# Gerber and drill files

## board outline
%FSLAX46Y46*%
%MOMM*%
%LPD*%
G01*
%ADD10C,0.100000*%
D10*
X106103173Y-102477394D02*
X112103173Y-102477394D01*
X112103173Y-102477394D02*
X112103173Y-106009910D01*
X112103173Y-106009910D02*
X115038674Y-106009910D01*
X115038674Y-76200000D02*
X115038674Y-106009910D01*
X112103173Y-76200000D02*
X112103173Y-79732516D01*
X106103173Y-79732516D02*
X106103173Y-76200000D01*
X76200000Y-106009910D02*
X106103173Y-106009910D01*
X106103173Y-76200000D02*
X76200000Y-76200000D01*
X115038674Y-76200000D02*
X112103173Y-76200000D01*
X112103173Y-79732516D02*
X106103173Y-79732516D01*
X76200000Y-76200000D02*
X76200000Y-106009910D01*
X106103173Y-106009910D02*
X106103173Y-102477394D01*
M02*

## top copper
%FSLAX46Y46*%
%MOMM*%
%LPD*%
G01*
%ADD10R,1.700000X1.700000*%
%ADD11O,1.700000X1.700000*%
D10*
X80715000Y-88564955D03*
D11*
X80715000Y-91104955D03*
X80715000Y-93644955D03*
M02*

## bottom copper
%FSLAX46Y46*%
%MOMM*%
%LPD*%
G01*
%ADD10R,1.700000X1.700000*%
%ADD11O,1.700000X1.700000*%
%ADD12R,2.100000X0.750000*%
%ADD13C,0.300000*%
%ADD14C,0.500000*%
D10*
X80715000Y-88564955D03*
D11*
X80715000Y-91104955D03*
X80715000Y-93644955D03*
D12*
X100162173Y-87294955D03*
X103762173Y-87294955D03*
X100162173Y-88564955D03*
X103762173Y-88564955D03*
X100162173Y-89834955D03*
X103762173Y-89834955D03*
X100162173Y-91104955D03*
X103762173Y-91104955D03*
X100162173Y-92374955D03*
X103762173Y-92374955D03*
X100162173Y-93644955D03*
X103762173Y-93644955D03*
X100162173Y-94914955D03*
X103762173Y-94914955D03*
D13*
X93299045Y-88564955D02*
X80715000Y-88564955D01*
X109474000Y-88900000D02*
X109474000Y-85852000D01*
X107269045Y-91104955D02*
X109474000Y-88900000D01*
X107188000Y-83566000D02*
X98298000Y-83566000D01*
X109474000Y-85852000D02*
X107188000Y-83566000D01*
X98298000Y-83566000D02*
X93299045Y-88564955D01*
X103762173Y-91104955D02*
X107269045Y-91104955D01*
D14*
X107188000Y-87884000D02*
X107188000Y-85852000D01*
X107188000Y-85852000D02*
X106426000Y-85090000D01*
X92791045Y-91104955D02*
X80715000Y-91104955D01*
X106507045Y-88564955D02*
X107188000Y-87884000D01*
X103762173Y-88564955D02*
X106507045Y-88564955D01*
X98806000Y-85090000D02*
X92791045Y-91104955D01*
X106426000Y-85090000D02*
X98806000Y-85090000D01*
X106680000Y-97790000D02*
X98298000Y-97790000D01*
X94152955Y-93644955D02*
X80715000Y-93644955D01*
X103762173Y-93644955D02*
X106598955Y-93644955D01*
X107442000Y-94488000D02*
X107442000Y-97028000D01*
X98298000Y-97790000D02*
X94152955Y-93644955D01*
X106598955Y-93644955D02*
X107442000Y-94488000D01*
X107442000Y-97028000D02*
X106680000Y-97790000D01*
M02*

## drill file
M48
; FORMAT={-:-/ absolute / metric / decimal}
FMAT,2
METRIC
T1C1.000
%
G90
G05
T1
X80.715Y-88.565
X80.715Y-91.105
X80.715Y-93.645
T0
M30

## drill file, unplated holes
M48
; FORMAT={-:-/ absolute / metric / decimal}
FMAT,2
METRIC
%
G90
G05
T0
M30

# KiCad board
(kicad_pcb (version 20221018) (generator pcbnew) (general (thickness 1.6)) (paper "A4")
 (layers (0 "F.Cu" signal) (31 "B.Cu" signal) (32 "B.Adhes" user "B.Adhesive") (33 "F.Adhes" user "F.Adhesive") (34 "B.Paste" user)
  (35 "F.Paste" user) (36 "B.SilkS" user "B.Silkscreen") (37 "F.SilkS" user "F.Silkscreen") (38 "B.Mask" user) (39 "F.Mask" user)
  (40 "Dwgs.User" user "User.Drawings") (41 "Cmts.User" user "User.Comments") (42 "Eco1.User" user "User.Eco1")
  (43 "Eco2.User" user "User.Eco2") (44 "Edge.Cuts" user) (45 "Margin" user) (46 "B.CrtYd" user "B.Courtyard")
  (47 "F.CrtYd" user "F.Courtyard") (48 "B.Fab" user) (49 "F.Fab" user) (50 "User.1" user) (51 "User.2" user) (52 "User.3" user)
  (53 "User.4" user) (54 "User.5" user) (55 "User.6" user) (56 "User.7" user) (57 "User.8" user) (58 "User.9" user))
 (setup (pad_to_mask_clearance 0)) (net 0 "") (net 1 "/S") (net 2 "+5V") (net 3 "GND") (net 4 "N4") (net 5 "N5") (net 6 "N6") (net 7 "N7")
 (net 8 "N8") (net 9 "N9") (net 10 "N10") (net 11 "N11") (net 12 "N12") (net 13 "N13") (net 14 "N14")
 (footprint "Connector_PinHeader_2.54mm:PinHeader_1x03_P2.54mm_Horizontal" (layer "F.Cu") (at 80.715 88.564955)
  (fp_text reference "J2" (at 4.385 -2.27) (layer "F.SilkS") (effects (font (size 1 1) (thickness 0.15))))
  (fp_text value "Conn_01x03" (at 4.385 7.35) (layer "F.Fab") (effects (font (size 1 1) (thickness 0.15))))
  (pad "1" thru_hole rect (at 0 0) (size 1.7 1.7) (drill 1) (layers "*.Cu" "*.Mask") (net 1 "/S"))
  (pad "2" thru_hole oval (at 0 2.54) (size 1.7 1.7) (drill 1) (layers "*.Cu" "*.Mask") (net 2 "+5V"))
  (pad "3" thru_hole oval (at 0 5.08) (size 1.7 1.7) (drill 1) (layers "*.Cu" "*.Mask") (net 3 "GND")))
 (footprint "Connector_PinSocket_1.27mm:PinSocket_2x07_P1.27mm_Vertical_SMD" (layer "B.Cu") (at 101.962173 91.104955 180)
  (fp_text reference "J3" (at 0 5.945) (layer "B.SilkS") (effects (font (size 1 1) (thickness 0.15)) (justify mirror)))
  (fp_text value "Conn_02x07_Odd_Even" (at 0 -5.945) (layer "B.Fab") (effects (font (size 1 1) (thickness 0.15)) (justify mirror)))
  (pad "1" smd rect (at 1.8 3.81 180) (size 2.1 0.75) (layers "B.Cu" "B.Paste" "B.Mask") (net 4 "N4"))
  (pad "2" smd rect (at -1.8 3.81 180) (size 2.1 0.75) (layers "B.Cu" "B.Paste" "B.Mask") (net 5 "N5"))
  (pad "3" smd rect (at 1.8 2.54 180) (size 2.1 0.75) (layers "B.Cu" "B.Paste" "B.Mask") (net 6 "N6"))
  (pad "4" smd rect (at -1.8 2.54 180) (size 2.1 0.75) (layers "B.Cu" "B.Paste" "B.Mask") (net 2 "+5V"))
  (pad "5" smd rect (at 1.8 1.27 180) (size 2.1 0.75) (layers "B.Cu" "B.Paste" "B.Mask") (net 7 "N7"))
  (pad "6" smd rect (at -1.8 1.27 180) (size 2.1 0.75) (layers "B.Cu" "B.Paste" "B.Mask") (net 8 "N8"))
  (pad "7" smd rect (at 1.8 0 180) (size 2.1 0.75) (layers "B.Cu" "B.Paste" "B.Mask") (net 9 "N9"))
  (pad "8" smd rect (at -1.8 0 180) (size 2.1 0.75) (layers "B.Cu" "B.Paste" "B.Mask") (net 1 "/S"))
  (pad "9" smd rect (at 1.8 -1.27 180) (size 2.1 0.75) (layers "B.Cu" "B.Paste" "B.Mask") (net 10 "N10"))
  (pad "10" smd rect (at -1.8 -1.27 180) (size 2.1 0.75) (layers "B.Cu" "B.Paste" "B.Mask") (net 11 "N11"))
  (pad "11" smd rect (at 1.8 -2.54 180) (size 2.1 0.75) (layers "B.Cu" "B.Paste" "B.Mask") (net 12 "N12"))
  (pad "12" smd rect (at -1.8 -2.54 180) (size 2.1 0.75) (layers "B.Cu" "B.Paste" "B.Mask") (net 3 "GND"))
  (pad "13" smd rect (at 1.8 -3.81 180) (size 2.1 0.75) (layers "B.Cu" "B.Paste" "B.Mask") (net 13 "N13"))
  (pad "14" smd rect (at -1.8 -3.81 180) (size 2.1 0.75) (layers "B.Cu" "B.Paste" "B.Mask") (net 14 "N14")))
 (gr_line (start 106.103173 102.477394) (end 112.103173 102.477394) (stroke (width 0.1) (type solid)) (layer "Edge.Cuts"))
 (gr_line (start 112.103173 102.477394) (end 112.103173 106.00991) (stroke (width 0.1) (type solid)) (layer "Edge.Cuts"))
 (gr_line (start 112.103173 106.00991) (end 115.038674 106.00991) (stroke (width 0.1) (type solid)) (layer "Edge.Cuts"))
 (gr_line (start 115.038674 76.2) (end 115.038674 106.00991) (stroke (width 0.1) (type solid)) (layer "Edge.Cuts"))
 (gr_line (start 112.103173 76.2) (end 112.103173 79.732516) (stroke (width 0.1) (type solid)) (layer "Edge.Cuts"))
 (gr_line (start 106.103173 79.732516) (end 106.103173 76.2) (stroke (width 0.1) (type solid)) (layer "Edge.Cuts"))
 (gr_line (start 76.2 106.00991) (end 106.103173 106.00991) (stroke (width 0.1) (type solid)) (layer "Edge.Cuts"))
 (gr_line (start 106.103173 76.2) (end 76.2 76.2) (stroke (width 0.1) (type solid)) (layer "Edge.Cuts"))
 (gr_line (start 115.038674 76.2) (end 112.103173 76.2) (stroke (width 0.1) (type solid)) (layer "Edge.Cuts"))
 (gr_line (start 112.103173 79.732516) (end 106.103173 79.732516) (stroke (width 0.1) (type solid)) (layer "Edge.Cuts"))
 (gr_line (start 76.2 76.2) (end 76.2 106.00991) (stroke (width 0.1) (type solid)) (layer "Edge.Cuts"))
 (gr_line (start 106.103173 106.00991) (end 106.103173 102.477394) (stroke (width 0.1) (type solid)) (layer "Edge.Cuts"))
 (segment (start 93.299045 88.564955) (end 80.715 88.564955) (width 0.3) (layer "B.Cu") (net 1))
 (segment (start 109.474 88.9) (end 109.474 85.852) (width 0.3) (layer "B.Cu") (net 1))
 (segment (start 107.269045 91.104955) (end 109.474 88.9) (width 0.3) (layer "B.Cu") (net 1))
 (segment (start 107.188 83.566) (end 98.298 83.566) (width 0.3) (layer "B.Cu") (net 1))
 (segment (start 109.474 85.852) (end 107.188 83.566) (width 0.3) (layer "B.Cu") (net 1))
 (segment (start 98.298 83.566) (end 93.299045 88.564955) (width 0.3) (layer "B.Cu") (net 1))
 (segment (start 103.762173 91.104955) (end 107.269045 91.104955) (width 0.3) (layer "B.Cu") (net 1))
 (segment (start 107.188 87.884) (end 107.188 85.852) (width 0.5) (layer "B.Cu") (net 2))
 (segment (start 107.188 85.852) (end 106.426 85.09) (width 0.5) (layer "B.Cu") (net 2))
 (segment (start 92.791045 91.104955) (end 80.715 91.104955) (width 0.5) (layer "B.Cu") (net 2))
 (segment (start 106.507045 88.564955) (end 107.188 87.884) (width 0.5) (layer "B.Cu") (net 2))
 (segment (start 103.762173 88.564955) (end 106.507045 88.564955) (width 0.5) (layer "B.Cu") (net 2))
 (segment (start 98.806 85.09) (end 92.791045 91.104955) (width 0.5) (layer "B.Cu") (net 2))
 (segment (start 106.426 85.09) (end 98.806 85.09) (width 0.5) (layer "B.Cu") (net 2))
 (segment (start 106.68 97.79) (end 98.298 97.79) (width 0.5) (layer "B.Cu") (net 3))
 (segment (start 94.152955 93.644955) (end 80.715 93.644955) (width 0.5) (layer "B.Cu") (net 3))
 (segment (start 103.762173 93.644955) (end 106.598955 93.644955) (width 0.5) (layer "B.Cu") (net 3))
 (segment (start 107.442 94.488) (end 107.442 97.028) (width 0.5) (layer "B.Cu") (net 3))
 (segment (start 98.298 97.79) (end 94.152955 93.644955) (width 0.5) (layer "B.Cu") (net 3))
 (segment (start 106.598955 93.644955) (end 107.442 94.488) (width 0.5) (layer "B.Cu") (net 3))
 (segment (start 107.442 97.028) (end 106.68 97.79) (width 0.5) (layer "B.Cu") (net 3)))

